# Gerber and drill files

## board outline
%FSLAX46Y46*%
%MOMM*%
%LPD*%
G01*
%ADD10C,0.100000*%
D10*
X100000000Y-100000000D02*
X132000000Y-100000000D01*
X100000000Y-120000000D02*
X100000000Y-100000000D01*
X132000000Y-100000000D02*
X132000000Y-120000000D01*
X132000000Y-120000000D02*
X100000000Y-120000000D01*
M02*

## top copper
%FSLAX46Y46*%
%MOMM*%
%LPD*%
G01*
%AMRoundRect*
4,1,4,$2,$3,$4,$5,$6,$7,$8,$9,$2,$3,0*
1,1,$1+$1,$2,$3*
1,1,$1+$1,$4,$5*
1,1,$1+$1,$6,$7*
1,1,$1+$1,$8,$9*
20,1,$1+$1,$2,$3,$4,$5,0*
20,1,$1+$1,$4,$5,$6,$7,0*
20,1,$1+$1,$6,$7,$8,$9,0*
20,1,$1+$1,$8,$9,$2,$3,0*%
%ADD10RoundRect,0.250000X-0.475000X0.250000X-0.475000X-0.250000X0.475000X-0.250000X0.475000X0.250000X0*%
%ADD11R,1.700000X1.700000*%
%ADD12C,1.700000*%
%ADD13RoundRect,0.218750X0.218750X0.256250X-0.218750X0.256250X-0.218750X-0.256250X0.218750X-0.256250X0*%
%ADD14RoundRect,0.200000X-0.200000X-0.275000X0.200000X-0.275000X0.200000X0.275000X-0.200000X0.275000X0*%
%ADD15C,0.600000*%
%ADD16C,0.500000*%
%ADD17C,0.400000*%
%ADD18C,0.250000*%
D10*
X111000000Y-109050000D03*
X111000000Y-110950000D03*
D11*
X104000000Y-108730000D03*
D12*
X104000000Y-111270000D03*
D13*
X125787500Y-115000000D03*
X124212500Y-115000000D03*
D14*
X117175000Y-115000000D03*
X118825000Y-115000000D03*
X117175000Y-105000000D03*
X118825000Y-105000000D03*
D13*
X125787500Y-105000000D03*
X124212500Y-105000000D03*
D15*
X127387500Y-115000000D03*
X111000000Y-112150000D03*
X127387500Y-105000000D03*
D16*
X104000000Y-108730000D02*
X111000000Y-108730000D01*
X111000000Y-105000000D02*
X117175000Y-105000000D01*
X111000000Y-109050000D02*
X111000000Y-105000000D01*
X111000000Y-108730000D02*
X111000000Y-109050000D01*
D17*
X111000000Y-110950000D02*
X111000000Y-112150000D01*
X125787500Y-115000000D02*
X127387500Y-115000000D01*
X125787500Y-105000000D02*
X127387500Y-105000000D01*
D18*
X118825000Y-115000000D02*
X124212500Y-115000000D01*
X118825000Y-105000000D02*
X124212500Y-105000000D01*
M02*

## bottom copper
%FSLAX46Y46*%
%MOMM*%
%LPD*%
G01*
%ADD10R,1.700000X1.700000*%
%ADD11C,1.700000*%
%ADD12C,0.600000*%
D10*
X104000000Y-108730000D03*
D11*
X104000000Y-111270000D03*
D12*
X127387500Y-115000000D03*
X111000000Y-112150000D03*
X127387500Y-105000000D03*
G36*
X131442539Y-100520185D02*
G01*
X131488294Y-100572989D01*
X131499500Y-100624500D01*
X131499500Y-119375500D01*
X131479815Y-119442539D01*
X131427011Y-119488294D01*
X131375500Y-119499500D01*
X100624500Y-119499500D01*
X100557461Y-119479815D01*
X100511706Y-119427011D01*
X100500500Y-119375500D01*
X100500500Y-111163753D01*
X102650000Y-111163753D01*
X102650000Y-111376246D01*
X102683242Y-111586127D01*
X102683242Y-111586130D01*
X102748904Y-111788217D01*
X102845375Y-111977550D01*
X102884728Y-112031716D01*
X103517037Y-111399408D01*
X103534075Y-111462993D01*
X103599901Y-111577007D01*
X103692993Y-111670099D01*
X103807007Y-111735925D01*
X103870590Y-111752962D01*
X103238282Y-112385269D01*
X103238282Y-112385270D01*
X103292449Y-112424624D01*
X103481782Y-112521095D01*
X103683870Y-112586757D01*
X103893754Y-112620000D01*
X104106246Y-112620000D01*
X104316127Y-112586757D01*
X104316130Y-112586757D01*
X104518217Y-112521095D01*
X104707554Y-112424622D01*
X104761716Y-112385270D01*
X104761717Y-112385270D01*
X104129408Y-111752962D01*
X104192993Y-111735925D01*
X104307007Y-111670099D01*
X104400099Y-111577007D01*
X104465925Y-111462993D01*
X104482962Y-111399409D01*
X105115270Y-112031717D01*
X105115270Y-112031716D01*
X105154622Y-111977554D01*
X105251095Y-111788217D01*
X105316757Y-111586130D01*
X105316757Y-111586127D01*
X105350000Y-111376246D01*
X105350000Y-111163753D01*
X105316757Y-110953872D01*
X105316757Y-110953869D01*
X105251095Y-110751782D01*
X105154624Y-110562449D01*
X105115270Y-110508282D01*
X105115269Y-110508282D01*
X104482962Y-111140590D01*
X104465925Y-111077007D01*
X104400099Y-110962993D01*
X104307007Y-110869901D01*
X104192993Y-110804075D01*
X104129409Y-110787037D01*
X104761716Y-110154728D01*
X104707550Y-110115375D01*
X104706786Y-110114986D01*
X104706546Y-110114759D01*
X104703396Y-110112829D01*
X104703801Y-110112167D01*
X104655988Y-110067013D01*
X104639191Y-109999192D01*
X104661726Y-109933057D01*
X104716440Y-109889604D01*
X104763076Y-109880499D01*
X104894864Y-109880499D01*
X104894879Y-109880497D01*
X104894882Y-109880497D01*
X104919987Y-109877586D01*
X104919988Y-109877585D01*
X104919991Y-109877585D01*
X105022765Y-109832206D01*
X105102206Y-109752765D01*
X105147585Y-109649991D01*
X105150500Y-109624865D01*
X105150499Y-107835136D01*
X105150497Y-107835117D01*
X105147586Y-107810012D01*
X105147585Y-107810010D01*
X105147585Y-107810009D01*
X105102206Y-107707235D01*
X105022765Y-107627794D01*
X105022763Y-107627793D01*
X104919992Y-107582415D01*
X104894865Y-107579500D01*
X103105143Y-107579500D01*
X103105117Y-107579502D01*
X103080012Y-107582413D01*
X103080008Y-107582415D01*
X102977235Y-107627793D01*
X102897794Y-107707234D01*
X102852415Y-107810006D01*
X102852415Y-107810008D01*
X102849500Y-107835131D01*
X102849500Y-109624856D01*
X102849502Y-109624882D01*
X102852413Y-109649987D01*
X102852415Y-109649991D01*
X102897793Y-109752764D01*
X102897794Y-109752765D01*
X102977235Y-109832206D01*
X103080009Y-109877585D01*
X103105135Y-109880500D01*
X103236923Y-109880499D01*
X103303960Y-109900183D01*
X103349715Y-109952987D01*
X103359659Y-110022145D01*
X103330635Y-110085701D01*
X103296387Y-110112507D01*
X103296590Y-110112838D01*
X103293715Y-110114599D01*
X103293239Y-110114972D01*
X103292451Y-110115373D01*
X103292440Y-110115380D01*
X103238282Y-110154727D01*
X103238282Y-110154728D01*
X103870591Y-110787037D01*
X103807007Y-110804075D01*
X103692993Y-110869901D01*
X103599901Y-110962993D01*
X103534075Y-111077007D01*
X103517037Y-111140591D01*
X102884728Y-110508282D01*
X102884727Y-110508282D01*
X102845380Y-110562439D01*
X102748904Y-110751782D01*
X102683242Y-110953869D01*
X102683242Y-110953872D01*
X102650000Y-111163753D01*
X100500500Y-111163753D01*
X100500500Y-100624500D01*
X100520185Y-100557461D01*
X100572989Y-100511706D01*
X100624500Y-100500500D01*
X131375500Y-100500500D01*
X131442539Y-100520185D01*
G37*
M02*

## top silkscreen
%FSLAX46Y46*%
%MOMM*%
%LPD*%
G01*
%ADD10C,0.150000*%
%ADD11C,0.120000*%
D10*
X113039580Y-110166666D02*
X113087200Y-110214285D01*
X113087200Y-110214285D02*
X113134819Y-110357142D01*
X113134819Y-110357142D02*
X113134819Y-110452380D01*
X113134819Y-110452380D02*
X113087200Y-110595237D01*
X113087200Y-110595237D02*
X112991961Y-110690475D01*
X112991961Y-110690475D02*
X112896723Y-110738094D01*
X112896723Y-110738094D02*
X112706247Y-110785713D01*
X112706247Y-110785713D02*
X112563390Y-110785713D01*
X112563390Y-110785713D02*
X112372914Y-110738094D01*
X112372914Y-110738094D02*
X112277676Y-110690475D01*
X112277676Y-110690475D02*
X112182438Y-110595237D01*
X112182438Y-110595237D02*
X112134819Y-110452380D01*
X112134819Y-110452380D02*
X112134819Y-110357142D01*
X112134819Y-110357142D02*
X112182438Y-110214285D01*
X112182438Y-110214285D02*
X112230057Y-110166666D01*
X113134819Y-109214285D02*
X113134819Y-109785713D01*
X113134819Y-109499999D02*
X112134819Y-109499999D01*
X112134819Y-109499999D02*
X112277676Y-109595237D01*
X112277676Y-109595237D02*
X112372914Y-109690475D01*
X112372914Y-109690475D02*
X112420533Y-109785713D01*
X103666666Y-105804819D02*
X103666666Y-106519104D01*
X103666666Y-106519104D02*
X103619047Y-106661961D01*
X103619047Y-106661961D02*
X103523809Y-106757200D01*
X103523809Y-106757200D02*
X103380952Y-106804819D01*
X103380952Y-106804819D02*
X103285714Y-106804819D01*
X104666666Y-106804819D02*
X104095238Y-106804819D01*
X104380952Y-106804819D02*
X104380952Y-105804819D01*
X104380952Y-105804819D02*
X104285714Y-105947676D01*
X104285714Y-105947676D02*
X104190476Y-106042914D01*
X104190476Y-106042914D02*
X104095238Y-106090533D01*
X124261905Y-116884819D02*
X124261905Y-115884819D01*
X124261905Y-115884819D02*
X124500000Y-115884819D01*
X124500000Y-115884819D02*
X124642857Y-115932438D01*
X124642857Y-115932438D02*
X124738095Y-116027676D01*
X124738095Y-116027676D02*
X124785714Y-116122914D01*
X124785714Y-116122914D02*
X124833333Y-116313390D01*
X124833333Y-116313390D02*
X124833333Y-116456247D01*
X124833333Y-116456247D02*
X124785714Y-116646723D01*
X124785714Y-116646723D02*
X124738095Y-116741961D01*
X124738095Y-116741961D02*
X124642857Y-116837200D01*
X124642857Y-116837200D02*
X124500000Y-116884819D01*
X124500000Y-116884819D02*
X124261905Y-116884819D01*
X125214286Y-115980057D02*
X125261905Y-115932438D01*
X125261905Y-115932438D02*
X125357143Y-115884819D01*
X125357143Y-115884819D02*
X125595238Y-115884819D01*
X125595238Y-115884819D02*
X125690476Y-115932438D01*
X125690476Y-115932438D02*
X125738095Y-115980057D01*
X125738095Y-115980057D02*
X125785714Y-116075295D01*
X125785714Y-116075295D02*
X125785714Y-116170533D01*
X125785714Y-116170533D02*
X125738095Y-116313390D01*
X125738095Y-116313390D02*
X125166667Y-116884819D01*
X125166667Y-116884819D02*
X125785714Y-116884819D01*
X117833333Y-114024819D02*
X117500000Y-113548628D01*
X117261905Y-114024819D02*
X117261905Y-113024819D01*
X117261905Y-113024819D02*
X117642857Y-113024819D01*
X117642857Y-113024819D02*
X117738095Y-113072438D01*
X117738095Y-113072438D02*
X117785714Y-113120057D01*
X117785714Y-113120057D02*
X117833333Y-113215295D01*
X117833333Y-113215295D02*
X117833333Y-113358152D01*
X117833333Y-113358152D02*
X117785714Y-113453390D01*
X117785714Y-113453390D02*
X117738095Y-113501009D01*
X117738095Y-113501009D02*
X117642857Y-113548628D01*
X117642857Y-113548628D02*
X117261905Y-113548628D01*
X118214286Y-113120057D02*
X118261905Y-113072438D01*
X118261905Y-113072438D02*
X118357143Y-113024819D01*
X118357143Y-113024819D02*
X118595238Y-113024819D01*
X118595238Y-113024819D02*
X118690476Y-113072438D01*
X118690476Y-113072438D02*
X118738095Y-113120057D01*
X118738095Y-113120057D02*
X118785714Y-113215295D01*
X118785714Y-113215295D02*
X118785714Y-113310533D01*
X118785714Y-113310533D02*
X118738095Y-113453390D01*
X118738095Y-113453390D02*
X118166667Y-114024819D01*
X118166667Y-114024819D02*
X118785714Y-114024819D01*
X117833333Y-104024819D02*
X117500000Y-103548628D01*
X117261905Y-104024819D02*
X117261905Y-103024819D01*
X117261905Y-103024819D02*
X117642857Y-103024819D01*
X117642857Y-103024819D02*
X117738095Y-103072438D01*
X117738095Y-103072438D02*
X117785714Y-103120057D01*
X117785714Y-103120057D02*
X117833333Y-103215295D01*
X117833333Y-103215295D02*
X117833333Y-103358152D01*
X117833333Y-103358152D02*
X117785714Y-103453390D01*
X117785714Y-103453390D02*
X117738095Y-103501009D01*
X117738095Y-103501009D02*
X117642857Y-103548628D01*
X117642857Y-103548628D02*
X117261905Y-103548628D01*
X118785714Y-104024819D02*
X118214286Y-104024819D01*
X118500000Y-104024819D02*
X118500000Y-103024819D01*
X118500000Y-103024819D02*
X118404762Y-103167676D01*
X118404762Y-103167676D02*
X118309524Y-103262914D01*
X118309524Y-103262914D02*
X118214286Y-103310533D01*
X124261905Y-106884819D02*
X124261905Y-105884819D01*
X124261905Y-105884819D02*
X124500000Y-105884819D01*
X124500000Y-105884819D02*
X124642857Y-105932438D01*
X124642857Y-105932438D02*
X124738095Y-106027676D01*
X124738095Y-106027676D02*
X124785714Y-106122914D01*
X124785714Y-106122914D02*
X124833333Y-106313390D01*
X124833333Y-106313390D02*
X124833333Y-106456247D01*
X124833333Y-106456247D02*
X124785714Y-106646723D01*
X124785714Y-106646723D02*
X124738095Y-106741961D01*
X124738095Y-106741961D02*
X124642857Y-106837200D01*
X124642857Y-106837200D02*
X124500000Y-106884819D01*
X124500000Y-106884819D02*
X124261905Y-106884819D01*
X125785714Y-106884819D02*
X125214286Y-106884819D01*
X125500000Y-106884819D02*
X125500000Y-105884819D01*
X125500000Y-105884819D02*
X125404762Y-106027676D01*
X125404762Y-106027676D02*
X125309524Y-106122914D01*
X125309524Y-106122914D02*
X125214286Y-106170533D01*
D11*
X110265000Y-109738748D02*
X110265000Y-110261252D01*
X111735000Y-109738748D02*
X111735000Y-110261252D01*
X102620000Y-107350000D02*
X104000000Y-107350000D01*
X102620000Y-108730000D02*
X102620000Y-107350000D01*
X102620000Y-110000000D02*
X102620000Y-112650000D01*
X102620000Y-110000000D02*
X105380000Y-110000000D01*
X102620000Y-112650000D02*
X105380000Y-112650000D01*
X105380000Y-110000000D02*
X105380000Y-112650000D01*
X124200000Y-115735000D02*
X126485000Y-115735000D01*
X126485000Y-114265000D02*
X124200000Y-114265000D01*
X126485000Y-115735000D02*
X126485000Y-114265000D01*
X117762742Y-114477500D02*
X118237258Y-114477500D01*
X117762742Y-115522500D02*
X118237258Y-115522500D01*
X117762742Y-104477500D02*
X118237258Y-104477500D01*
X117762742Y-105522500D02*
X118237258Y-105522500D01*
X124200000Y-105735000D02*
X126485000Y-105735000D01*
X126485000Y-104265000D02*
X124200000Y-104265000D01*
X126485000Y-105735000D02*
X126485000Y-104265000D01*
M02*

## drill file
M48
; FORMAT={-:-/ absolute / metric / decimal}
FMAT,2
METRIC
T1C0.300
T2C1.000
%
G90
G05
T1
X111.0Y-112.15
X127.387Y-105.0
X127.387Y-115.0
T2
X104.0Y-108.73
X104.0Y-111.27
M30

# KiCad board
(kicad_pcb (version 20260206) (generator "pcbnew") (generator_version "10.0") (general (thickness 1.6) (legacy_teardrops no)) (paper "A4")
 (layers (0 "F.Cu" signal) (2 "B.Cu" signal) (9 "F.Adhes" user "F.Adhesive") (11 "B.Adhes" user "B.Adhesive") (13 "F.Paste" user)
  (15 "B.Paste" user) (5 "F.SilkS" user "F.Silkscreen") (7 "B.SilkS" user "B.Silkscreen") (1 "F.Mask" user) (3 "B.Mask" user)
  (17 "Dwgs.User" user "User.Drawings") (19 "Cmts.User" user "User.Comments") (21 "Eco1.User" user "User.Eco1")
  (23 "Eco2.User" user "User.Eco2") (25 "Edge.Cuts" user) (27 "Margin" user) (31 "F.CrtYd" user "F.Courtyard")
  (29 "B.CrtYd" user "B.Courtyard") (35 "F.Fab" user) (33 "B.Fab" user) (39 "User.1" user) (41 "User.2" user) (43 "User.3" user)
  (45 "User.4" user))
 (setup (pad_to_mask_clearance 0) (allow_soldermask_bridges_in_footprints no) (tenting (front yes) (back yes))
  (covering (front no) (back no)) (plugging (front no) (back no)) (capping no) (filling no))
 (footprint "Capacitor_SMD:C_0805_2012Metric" (layer "F.Cu") (at 111 110 -90)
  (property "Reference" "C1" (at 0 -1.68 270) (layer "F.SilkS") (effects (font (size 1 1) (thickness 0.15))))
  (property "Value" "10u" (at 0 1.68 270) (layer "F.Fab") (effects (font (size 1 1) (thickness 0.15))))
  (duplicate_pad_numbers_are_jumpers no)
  (fp_line (start -0.261252 0.735) (end 0.261252 0.735) (stroke (width 0.12) (type solid)) (layer "F.SilkS"))
  (fp_line (start -0.261252 -0.735) (end 0.261252 -0.735) (stroke (width 0.12) (type solid)) (layer "F.SilkS"))
  (pad "1" smd roundrect (at -0.95 0 270) (size 1 1.45) (layers "F.Cu" "F.Mask" "F.Paste") (roundrect_rratio 0.25) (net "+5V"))
  (pad "2" smd roundrect (at 0.95 0 270) (size 1 1.45) (layers "F.Cu" "F.Mask" "F.Paste") (roundrect_rratio 0.25) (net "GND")))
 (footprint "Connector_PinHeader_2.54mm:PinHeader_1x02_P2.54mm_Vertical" (layer "F.Cu") (at 104 108.73)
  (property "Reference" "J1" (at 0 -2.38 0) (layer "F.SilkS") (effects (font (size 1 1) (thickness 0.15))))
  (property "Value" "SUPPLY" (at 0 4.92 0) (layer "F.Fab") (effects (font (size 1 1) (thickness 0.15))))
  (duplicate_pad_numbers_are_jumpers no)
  (fp_line (start -1.38 -1.38) (end 0 -1.38) (stroke (width 0.12) (type solid)) (layer "F.SilkS"))
  (fp_line (start -1.38 0) (end -1.38 -1.38) (stroke (width 0.12) (type solid)) (layer "F.SilkS"))
  (fp_line (start -1.38 1.27) (end -1.38 3.92) (stroke (width 0.12) (type solid)) (layer "F.SilkS"))
  (fp_line (start -1.38 1.27) (end 1.38 1.27) (stroke (width 0.12) (type solid)) (layer "F.SilkS"))
  (fp_line (start -1.38 3.92) (end 1.38 3.92) (stroke (width 0.12) (type solid)) (layer "F.SilkS"))
  (fp_line (start 1.38 1.27) (end 1.38 3.92) (stroke (width 0.12) (type solid)) (layer "F.SilkS"))
  (pad "1" thru_hole rect (at 0 0) (size 1.7 1.7) (drill 1) (layers "*.Cu" "*.Mask") (remove_unused_layers no) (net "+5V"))
  (pad "2" thru_hole circle (at 0 2.54) (size 1.7 1.7) (drill 1) (layers "*.Cu" "*.Mask") (remove_unused_layers no) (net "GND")))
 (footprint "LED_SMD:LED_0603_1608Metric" (layer "F.Cu") (at 125 115 180)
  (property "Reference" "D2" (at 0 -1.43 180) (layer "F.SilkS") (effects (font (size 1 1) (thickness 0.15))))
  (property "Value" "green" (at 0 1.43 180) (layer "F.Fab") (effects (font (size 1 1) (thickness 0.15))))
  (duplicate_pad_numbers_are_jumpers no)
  (fp_line (start 0.8 -0.735) (end -1.485 -0.735) (stroke (width 0.12) (type solid)) (layer "F.SilkS"))
  (fp_line (start -1.485 0.735) (end 0.8 0.735) (stroke (width 0.12) (type solid)) (layer "F.SilkS"))
  (fp_line (start -1.485 -0.735) (end -1.485 0.735) (stroke (width 0.12) (type solid)) (layer "F.SilkS"))
  (pad "1" smd roundrect (at -0.7875 0 180) (size 0.875 0.95) (layers "F.Cu" "F.Mask" "F.Paste") (roundrect_rratio 0.25) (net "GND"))
  (pad "2" smd roundrect (at 0.7875 0 180) (size 0.875 0.95) (layers "F.Cu" "F.Mask" "F.Paste") (roundrect_rratio 0.25) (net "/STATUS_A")))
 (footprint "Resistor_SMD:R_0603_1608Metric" (layer "F.Cu") (at 118 115)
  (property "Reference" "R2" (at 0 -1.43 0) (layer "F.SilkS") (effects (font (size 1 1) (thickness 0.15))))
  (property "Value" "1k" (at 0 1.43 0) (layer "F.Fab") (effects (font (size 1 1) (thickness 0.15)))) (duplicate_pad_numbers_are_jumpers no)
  (fp_line (start -0.237258 -0.5225) (end 0.237258 -0.5225) (stroke (width 0.12) (type solid)) (layer "F.SilkS"))
  (fp_line (start -0.237258 0.5225) (end 0.237258 0.5225) (stroke (width 0.12) (type solid)) (layer "F.SilkS"))
  (pad "1" smd roundrect (at -0.825 0) (size 0.8 0.95) (layers "F.Cu" "F.Mask" "F.Paste") (roundrect_rratio 0.25) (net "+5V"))
  (pad "2" smd roundrect (at 0.825 0) (size 0.8 0.95) (layers "F.Cu" "F.Mask" "F.Paste") (roundrect_rratio 0.25) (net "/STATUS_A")))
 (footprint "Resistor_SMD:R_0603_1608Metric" (layer "F.Cu") (at 118 105)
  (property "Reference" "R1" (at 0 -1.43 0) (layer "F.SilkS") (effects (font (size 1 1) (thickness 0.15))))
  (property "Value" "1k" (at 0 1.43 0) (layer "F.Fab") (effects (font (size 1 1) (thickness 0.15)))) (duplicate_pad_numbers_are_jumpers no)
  (fp_line (start -0.237258 -0.5225) (end 0.237258 -0.5225) (stroke (width 0.12) (type solid)) (layer "F.SilkS"))
  (fp_line (start -0.237258 0.5225) (end 0.237258 0.5225) (stroke (width 0.12) (type solid)) (layer "F.SilkS"))
  (pad "1" smd roundrect (at -0.825 0) (size 0.8 0.95) (layers "F.Cu" "F.Mask" "F.Paste") (roundrect_rratio 0.25) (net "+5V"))
  (pad "2" smd roundrect (at 0.825 0) (size 0.8 0.95) (layers "F.Cu" "F.Mask" "F.Paste") (roundrect_rratio 0.25) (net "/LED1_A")))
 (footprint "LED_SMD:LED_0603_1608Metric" (layer "F.Cu") (at 125 105 180)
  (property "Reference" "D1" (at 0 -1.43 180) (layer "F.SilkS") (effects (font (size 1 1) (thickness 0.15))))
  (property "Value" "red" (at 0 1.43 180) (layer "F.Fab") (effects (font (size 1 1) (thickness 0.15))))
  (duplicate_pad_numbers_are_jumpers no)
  (fp_line (start 0.8 -0.735) (end -1.485 -0.735) (stroke (width 0.12) (type solid)) (layer "F.SilkS"))
  (fp_line (start -1.485 0.735) (end 0.8 0.735) (stroke (width 0.12) (type solid)) (layer "F.SilkS"))
  (fp_line (start -1.485 -0.735) (end -1.485 0.735) (stroke (width 0.12) (type solid)) (layer "F.SilkS"))
  (pad "1" smd roundrect (at -0.7875 0 180) (size 0.875 0.95) (layers "F.Cu" "F.Mask" "F.Paste") (roundrect_rratio 0.25) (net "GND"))
  (pad "2" smd roundrect (at 0.7875 0 180) (size 0.875 0.95) (layers "F.Cu" "F.Mask" "F.Paste") (roundrect_rratio 0.25) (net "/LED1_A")))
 (gr_line (start 100 100) (end 132 100) (stroke (width 0.1) (type default)) (layer "Edge.Cuts"))
 (gr_line (start 100 120) (end 100 100) (stroke (width 0.1) (type default)) (layer "Edge.Cuts"))
 (gr_line (start 132 100) (end 132 120) (stroke (width 0.1) (type default)) (layer "Edge.Cuts"))
 (gr_line (start 132 120) (end 100 120) (stroke (width 0.1) (type default)) (layer "Edge.Cuts"))
 (segment (start 104 108.73) (end 111 108.73) (width 0.5) (layer "F.Cu") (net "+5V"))
 (segment (start 111 105) (end 117.175 105) (width 0.5) (layer "F.Cu") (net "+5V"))
 (segment (start 111 109.05) (end 111 105) (width 0.5) (layer "F.Cu") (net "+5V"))
 (segment (start 111 108.73) (end 111 109.05) (width 0.5) (layer "F.Cu") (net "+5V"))
 (segment (start 111 110.95) (end 111 112.15) (width 0.4) (layer "F.Cu") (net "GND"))
 (segment (start 125.7875 115) (end 127.3875 115) (width 0.4) (layer "F.Cu") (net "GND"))
 (segment (start 125.7875 105) (end 127.3875 105) (width 0.4) (layer "F.Cu") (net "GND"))
 (via (at 127.3875 115) (size 0.6) (drill 0.3) (layers "F.Cu" "B.Cu") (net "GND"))
 (via (at 111 112.15) (size 0.6) (drill 0.3) (layers "F.Cu" "B.Cu") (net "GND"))
 (via (at 127.3875 105) (size 0.6) (drill 0.3) (layers "F.Cu" "B.Cu") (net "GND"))
 (segment (start 118.825 115) (end 124.2125 115) (width 0.25) (layer "F.Cu") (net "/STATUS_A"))
 (segment (start 118.825 105) (end 124.2125 105) (width 0.25) (layer "F.Cu") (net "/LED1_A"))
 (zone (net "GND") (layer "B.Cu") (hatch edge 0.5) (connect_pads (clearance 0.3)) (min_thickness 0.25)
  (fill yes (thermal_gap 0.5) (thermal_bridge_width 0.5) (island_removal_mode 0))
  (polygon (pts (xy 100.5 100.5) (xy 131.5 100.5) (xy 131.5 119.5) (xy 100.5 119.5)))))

